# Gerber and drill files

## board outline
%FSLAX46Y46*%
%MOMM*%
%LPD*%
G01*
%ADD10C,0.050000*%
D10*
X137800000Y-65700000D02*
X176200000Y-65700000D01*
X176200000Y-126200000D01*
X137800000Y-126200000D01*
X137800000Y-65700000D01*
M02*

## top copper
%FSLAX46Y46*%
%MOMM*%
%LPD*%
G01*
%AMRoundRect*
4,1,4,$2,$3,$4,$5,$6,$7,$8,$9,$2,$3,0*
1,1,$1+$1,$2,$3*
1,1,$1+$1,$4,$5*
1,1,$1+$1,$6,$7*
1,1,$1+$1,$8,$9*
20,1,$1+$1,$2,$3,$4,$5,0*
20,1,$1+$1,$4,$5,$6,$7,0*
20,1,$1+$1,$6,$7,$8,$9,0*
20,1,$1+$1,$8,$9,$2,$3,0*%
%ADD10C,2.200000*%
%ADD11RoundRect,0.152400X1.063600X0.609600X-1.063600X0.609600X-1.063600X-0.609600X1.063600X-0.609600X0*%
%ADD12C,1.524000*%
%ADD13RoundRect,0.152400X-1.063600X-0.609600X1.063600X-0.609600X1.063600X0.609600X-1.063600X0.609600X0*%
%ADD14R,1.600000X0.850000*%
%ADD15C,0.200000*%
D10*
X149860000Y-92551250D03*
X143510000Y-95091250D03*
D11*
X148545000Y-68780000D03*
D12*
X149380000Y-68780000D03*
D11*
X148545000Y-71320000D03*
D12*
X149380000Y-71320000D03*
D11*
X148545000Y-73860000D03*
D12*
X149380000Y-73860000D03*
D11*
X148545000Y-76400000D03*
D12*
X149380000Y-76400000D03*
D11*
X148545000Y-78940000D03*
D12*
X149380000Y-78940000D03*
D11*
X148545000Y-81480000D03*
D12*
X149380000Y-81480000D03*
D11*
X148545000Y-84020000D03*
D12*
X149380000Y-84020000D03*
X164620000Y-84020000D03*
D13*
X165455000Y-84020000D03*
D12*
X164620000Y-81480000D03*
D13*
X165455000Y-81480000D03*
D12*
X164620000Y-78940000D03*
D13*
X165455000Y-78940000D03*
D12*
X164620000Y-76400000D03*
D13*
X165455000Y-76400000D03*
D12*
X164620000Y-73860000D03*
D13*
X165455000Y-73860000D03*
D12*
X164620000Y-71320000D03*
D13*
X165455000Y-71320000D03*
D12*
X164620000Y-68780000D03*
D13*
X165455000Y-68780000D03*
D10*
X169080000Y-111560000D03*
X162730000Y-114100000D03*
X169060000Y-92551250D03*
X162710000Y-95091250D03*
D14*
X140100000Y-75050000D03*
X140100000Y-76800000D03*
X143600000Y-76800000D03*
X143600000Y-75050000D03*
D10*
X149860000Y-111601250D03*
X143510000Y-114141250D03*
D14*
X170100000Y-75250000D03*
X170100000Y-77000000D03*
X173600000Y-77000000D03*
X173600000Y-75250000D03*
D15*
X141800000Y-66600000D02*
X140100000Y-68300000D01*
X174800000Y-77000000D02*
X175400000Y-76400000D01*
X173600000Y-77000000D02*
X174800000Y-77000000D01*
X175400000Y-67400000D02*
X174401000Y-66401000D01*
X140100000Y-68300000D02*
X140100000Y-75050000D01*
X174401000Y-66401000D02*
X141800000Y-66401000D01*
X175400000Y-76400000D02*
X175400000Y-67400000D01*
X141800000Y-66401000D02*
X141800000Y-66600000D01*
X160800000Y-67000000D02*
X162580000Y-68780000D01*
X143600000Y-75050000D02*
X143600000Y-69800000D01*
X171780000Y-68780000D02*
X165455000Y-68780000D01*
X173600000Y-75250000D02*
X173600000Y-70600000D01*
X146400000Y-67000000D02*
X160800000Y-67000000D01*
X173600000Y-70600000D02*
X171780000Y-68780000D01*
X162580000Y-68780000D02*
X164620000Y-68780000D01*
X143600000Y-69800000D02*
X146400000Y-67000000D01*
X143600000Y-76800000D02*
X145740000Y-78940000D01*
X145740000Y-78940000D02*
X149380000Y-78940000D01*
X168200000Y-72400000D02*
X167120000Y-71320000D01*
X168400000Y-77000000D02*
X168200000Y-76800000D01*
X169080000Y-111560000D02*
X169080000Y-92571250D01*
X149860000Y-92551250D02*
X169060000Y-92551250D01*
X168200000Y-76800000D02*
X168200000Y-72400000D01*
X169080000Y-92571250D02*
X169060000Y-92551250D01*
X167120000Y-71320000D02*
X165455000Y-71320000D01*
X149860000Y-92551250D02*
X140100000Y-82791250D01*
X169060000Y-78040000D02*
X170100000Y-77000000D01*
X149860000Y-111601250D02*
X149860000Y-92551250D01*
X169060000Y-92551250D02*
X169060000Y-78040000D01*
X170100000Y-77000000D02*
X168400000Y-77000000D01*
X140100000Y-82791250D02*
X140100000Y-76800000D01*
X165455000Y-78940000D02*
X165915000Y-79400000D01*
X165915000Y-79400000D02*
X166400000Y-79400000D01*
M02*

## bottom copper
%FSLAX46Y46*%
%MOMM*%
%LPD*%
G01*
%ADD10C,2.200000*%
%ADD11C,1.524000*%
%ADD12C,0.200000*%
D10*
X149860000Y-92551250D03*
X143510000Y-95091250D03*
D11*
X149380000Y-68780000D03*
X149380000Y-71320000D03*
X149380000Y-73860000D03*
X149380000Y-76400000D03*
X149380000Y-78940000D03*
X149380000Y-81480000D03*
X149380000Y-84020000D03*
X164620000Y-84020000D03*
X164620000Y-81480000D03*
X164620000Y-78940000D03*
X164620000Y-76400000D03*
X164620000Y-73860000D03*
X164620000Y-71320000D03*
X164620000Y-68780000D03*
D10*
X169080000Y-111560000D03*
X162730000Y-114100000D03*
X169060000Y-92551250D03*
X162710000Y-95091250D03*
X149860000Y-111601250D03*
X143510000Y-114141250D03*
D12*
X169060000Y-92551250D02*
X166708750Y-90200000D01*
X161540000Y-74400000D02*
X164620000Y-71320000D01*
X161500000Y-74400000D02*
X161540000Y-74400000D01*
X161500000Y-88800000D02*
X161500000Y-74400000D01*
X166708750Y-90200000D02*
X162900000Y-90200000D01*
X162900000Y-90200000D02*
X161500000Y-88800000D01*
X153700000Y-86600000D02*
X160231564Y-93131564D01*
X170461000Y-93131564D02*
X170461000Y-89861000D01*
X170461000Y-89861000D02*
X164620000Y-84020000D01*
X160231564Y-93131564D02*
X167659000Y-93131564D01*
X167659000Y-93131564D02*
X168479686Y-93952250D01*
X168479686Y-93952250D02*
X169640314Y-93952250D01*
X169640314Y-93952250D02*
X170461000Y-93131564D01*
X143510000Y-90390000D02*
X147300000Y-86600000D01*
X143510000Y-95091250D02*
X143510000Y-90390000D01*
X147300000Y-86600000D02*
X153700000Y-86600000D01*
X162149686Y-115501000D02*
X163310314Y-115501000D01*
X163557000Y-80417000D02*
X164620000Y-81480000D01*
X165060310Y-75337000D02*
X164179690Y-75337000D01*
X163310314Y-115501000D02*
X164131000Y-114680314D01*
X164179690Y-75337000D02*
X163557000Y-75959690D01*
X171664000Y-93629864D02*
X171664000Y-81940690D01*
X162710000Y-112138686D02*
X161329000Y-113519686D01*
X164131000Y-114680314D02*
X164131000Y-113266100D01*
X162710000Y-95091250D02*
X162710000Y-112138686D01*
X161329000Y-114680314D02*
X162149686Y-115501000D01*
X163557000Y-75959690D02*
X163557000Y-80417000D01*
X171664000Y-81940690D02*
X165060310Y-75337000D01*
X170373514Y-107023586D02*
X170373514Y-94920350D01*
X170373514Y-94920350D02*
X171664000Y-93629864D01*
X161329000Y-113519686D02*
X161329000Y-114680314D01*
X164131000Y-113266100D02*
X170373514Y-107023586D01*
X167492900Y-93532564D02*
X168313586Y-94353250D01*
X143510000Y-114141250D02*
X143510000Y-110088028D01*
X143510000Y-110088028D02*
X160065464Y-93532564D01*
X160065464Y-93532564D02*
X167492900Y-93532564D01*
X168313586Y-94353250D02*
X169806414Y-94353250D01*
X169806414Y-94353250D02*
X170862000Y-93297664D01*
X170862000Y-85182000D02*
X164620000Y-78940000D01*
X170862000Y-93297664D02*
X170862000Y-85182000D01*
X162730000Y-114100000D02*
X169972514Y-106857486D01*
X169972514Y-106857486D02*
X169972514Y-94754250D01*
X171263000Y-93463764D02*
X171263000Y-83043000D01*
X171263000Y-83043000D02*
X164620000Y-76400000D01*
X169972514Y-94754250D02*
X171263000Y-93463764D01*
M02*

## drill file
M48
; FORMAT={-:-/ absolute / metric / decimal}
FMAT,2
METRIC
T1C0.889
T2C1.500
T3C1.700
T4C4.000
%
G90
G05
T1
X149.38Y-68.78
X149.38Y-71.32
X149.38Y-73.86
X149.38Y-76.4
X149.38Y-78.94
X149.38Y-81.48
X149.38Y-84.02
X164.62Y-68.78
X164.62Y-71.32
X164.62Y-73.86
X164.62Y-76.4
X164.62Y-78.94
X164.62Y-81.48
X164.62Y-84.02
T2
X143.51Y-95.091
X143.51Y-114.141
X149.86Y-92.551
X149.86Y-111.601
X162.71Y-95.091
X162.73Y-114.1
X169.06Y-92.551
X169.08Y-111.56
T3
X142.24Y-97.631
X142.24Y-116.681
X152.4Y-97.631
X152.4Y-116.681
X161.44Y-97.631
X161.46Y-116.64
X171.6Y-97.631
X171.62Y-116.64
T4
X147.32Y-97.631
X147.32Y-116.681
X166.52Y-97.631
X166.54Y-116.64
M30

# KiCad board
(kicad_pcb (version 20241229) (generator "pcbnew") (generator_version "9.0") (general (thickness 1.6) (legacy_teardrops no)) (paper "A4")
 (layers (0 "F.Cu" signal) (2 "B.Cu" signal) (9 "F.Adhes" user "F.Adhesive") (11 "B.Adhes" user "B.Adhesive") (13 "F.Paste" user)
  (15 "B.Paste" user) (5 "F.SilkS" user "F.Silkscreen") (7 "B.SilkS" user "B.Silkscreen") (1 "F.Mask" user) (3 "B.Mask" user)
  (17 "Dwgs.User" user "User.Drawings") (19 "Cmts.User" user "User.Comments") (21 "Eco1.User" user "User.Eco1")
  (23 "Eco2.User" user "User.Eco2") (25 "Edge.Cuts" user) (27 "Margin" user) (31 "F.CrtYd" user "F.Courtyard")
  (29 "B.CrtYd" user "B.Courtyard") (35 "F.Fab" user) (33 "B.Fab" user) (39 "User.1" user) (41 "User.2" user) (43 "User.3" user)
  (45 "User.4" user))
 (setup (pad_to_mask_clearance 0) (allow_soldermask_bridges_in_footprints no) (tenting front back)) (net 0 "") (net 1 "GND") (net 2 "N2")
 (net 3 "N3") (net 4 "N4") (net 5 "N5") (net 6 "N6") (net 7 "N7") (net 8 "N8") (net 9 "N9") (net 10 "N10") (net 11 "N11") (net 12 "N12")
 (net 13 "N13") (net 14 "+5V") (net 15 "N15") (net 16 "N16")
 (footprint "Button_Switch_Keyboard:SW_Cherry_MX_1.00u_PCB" (layer "F.Cu") (at 149.86 92.55125)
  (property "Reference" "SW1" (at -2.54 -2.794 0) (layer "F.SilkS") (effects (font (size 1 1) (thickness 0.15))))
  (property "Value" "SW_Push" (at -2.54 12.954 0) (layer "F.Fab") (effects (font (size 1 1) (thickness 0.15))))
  (pad "" np_thru_hole circle (at -7.62 5.08) (size 1.7 1.7) (drill 1.7) (layers "*.Cu" "*.Mask"))
  (pad "" np_thru_hole circle (at -2.54 5.08) (size 4 4) (drill 4) (layers "*.Cu" "*.Mask"))
  (pad "" np_thru_hole circle (at 2.54 5.08) (size 1.7 1.7) (drill 1.7) (layers "*.Cu" "*.Mask"))
  (pad "1" thru_hole circle (at 0 0) (size 2.2 2.2) (drill 1.5) (layers "*.Cu" "*.Mask") (remove_unused_layers no) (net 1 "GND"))
  (pad "2" thru_hole circle (at -6.35 2.54) (size 2.2 2.2) (drill 1.5) (layers "*.Cu" "*.Mask") (remove_unused_layers no) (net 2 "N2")))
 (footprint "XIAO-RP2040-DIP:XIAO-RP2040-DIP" (layer "F.Cu") (at 157 76.4)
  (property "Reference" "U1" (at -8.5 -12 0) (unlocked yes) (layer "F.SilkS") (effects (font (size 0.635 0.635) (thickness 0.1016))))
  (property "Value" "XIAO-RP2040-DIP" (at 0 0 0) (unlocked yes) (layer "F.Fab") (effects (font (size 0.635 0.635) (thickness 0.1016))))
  (pad "1" smd roundrect (at -8.455 -7.62 180) (size 2.432 1.524) (layers "F.Cu" "F.Mask") (roundrect_rratio 0.1) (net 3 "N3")
   (thermal_bridge_angle 45))
  (pad "1" thru_hole circle (at -7.62 -7.62 180) (size 1.524 1.524) (drill 0.889) (layers "*.Cu" "*.Mask") (remove_unused_layers no)
   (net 3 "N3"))
  (pad "2" smd roundrect (at -8.455 -5.08 180) (size 2.432 1.524) (layers "F.Cu" "F.Mask") (roundrect_rratio 0.1) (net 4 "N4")
   (thermal_bridge_angle 45))
  (pad "2" thru_hole circle (at -7.62 -5.08 180) (size 1.524 1.524) (drill 0.889) (layers "*.Cu" "*.Mask") (remove_unused_layers no)
   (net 4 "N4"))
  (pad "3" smd roundrect (at -8.455 -2.54 180) (size 2.432 1.524) (layers "F.Cu" "F.Mask") (roundrect_rratio 0.1) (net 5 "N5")
   (thermal_bridge_angle 45))
  (pad "3" thru_hole circle (at -7.62 -2.54 180) (size 1.524 1.524) (drill 0.889) (layers "*.Cu" "*.Mask") (remove_unused_layers no)
   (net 5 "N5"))
  (pad "4" smd roundrect (at -8.455 0 180) (size 2.432 1.524) (layers "F.Cu" "F.Mask") (roundrect_rratio 0.1) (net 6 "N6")
   (thermal_bridge_angle 45))
  (pad "4" thru_hole circle (at -7.62 0 180) (size 1.524 1.524) (drill 0.889) (layers "*.Cu" "*.Mask") (remove_unused_layers no)
   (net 6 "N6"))
  (pad "5" smd roundrect (at -8.455 2.54 180) (size 2.432 1.524) (layers "F.Cu" "F.Mask") (roundrect_rratio 0.1) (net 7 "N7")
   (thermal_bridge_angle 45))
  (pad "5" thru_hole circle (at -7.62 2.54 180) (size 1.524 1.524) (drill 0.889) (layers "*.Cu" "*.Mask") (remove_unused_layers no)
   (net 7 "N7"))
  (pad "6" smd roundrect (at -8.455 5.08 180) (size 2.432 1.524) (layers "F.Cu" "F.Mask") (roundrect_rratio 0.1) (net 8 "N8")
   (thermal_bridge_angle 45))
  (pad "6" thru_hole circle (at -7.62 5.08 180) (size 1.524 1.524) (drill 0.889) (layers "*.Cu" "*.Mask") (remove_unused_layers no)
   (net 8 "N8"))
  (pad "7" smd roundrect (at -8.455 7.62 180) (size 2.432 1.524) (layers "F.Cu" "F.Mask") (roundrect_rratio 0.1) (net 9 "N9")
   (thermal_bridge_angle 45))
  (pad "7" thru_hole circle (at -7.62 7.62 180) (size 1.524 1.524) (drill 0.889) (layers "*.Cu" "*.Mask") (remove_unused_layers no)
   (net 9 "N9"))
  (pad "8" thru_hole circle (at 7.62 7.62) (size 1.524 1.524) (drill 0.889) (layers "*.Cu" "*.Mask") (remove_unused_layers no) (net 2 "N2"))
  (pad "8" smd roundrect (at 8.455 7.62) (size 2.432 1.524) (layers "F.Cu" "F.Mask") (roundrect_rratio 0.1) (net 2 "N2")
   (thermal_bridge_angle 45))
  (pad "9" thru_hole circle (at 7.62 5.08) (size 1.524 1.524) (drill 0.889) (layers "*.Cu" "*.Mask") (remove_unused_layers no)
   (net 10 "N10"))
  (pad "9" smd roundrect (at 8.455 5.08) (size 2.432 1.524) (layers "F.Cu" "F.Mask") (roundrect_rratio 0.1) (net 10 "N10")
   (thermal_bridge_angle 45))
  (pad "10" thru_hole circle (at 7.62 2.54) (size 1.524 1.524) (drill 0.889) (layers "*.Cu" "*.Mask") (remove_unused_layers no)
   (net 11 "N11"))
  (pad "10" smd roundrect (at 8.455 2.54) (size 2.432 1.524) (layers "F.Cu" "F.Mask") (roundrect_rratio 0.1) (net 11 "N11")
   (thermal_bridge_angle 45))
  (pad "11" thru_hole circle (at 7.62 0) (size 1.524 1.524) (drill 0.889) (layers "*.Cu" "*.Mask") (remove_unused_layers no) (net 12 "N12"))
  (pad "11" smd roundrect (at 8.455 0) (size 2.432 1.524) (layers "F.Cu" "F.Mask") (roundrect_rratio 0.1) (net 12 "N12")
   (thermal_bridge_angle 45))
  (pad "12" thru_hole circle (at 7.62 -2.54) (size 1.524 1.524) (drill 0.889) (layers "*.Cu" "*.Mask") (remove_unused_layers no)
   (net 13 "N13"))
  (pad "12" smd roundrect (at 8.455 -2.54) (size 2.432 1.524) (layers "F.Cu" "F.Mask") (roundrect_rratio 0.1) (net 13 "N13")
   (thermal_bridge_angle 45))
  (pad "13" thru_hole circle (at 7.62 -5.08) (size 1.524 1.524) (drill 0.889) (layers "*.Cu" "*.Mask") (remove_unused_layers no)
   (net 1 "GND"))
  (pad "13" smd roundrect (at 8.455 -5.08) (size 2.432 1.524) (layers "F.Cu" "F.Mask") (roundrect_rratio 0.1) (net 1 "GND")
   (thermal_bridge_angle 45))
  (pad "14" thru_hole circle (at 7.62 -7.62) (size 1.524 1.524) (drill 0.889) (layers "*.Cu" "*.Mask") (remove_unused_layers no)
   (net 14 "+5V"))
  (pad "14" smd roundrect (at 8.455 -7.62) (size 2.432 1.524) (layers "F.Cu" "F.Mask") (roundrect_rratio 0.1) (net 14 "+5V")
   (thermal_bridge_angle 45)))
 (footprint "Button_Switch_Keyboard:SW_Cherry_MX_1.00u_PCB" (layer "F.Cu") (at 169.08 111.56)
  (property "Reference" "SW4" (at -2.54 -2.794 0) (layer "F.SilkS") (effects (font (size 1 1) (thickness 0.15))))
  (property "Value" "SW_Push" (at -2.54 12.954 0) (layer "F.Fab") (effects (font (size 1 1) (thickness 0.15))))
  (pad "" np_thru_hole circle (at -7.62 5.08) (size 1.7 1.7) (drill 1.7) (layers "*.Cu" "*.Mask"))
  (pad "" np_thru_hole circle (at -2.54 5.08) (size 4 4) (drill 4) (layers "*.Cu" "*.Mask"))
  (pad "" np_thru_hole circle (at 2.54 5.08) (size 1.7 1.7) (drill 1.7) (layers "*.Cu" "*.Mask"))
  (pad "1" thru_hole circle (at 0 0) (size 2.2 2.2) (drill 1.5) (layers "*.Cu" "*.Mask") (remove_unused_layers no) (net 1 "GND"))
  (pad "2" thru_hole circle (at -6.35 2.54) (size 2.2 2.2) (drill 1.5) (layers "*.Cu" "*.Mask") (remove_unused_layers no) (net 12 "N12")))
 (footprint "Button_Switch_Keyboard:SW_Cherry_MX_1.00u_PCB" (layer "F.Cu") (at 169.06 92.55125)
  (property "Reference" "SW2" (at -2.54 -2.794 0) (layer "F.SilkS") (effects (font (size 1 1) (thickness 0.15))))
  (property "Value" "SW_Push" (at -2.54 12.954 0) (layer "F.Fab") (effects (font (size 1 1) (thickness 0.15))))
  (pad "" np_thru_hole circle (at -7.62 5.08) (size 1.7 1.7) (drill 1.7) (layers "*.Cu" "*.Mask"))
  (pad "" np_thru_hole circle (at -2.54 5.08) (size 4 4) (drill 4) (layers "*.Cu" "*.Mask"))
  (pad "" np_thru_hole circle (at 2.54 5.08) (size 1.7 1.7) (drill 1.7) (layers "*.Cu" "*.Mask"))
  (pad "1" thru_hole circle (at 0 0) (size 2.2 2.2) (drill 1.5) (layers "*.Cu" "*.Mask") (remove_unused_layers no) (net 1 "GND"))
  (pad "2" thru_hole circle (at -6.35 2.54) (size 2.2 2.2) (drill 1.5) (layers "*.Cu" "*.Mask") (remove_unused_layers no) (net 10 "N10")))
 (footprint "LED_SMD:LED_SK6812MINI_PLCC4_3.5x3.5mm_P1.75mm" (layer "F.Cu") (at 141.85 75.925)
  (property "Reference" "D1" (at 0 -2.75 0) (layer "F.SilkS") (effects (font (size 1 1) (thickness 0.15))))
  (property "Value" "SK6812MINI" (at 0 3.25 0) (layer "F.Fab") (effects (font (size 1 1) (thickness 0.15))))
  (pad "1" smd rect (at -1.75 -0.875) (size 1.6 0.85) (layers "F.Cu" "F.Mask" "F.Paste") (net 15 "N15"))
  (pad "2" smd rect (at -1.75 0.875) (size 1.6 0.85) (layers "F.Cu" "F.Mask" "F.Paste") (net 1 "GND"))
  (pad "3" smd rect (at 1.75 0.875) (size 1.6 0.85) (layers "F.Cu" "F.Mask" "F.Paste") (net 7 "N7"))
  (pad "4" smd rect (at 1.75 -0.875) (size 1.6 0.85) (layers "F.Cu" "F.Mask" "F.Paste") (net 14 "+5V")))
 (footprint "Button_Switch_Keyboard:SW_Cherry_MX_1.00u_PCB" (layer "F.Cu") (at 149.86 111.60125)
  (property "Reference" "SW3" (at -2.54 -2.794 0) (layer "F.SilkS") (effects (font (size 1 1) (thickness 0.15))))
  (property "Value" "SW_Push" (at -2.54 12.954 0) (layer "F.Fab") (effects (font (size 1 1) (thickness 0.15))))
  (pad "" np_thru_hole circle (at -7.62 5.08) (size 1.7 1.7) (drill 1.7) (layers "*.Cu" "*.Mask"))
  (pad "" np_thru_hole circle (at -2.54 5.08) (size 4 4) (drill 4) (layers "*.Cu" "*.Mask"))
  (pad "" np_thru_hole circle (at 2.54 5.08) (size 1.7 1.7) (drill 1.7) (layers "*.Cu" "*.Mask"))
  (pad "1" thru_hole circle (at 0 0) (size 2.2 2.2) (drill 1.5) (layers "*.Cu" "*.Mask") (remove_unused_layers no) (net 1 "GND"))
  (pad "2" thru_hole circle (at -6.35 2.54) (size 2.2 2.2) (drill 1.5) (layers "*.Cu" "*.Mask") (remove_unused_layers no) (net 11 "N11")))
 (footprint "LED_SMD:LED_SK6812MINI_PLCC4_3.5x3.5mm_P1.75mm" (layer "F.Cu") (at 171.85 76.125)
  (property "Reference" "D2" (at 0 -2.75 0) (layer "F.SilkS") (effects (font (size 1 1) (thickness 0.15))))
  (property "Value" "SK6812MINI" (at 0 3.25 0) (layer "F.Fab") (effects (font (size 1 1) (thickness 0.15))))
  (pad "1" smd rect (at -1.75 -0.875) (size 1.6 0.85) (layers "F.Cu" "F.Mask" "F.Paste") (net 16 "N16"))
  (pad "2" smd rect (at -1.75 0.875) (size 1.6 0.85) (layers "F.Cu" "F.Mask" "F.Paste") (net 1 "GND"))
  (pad "3" smd rect (at 1.75 0.875) (size 1.6 0.85) (layers "F.Cu" "F.Mask" "F.Paste") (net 15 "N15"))
  (pad "4" smd rect (at 1.75 -0.875) (size 1.6 0.85) (layers "F.Cu" "F.Mask" "F.Paste") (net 14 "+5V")))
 (gr_rect (start 137.8 65.7) (end 176.2 126.2) (stroke (width 0.05) (type default)) (fill no) (layer "Edge.Cuts"))
 (segment (start 141.8 66.6) (end 140.1 68.3) (width 0.2) (layer "F.Cu") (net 15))
 (segment (start 174.8 77) (end 175.4 76.4) (width 0.2) (layer "F.Cu") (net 15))
 (segment (start 173.6 77) (end 174.8 77) (width 0.2) (layer "F.Cu") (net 15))
 (segment (start 175.4 67.4) (end 174.401 66.401) (width 0.2) (layer "F.Cu") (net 15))
 (segment (start 140.1 68.3) (end 140.1 75.05) (width 0.2) (layer "F.Cu") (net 15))
 (segment (start 174.401 66.401) (end 141.8 66.401) (width 0.2) (layer "F.Cu") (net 15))
 (segment (start 175.4 76.4) (end 175.4 67.4) (width 0.2) (layer "F.Cu") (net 15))
 (segment (start 141.8 66.401) (end 141.8 66.6) (width 0.2) (layer "F.Cu") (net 15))
 (segment (start 160.8 67) (end 162.58 68.78) (width 0.2) (layer "F.Cu") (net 14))
 (segment (start 143.6 75.05) (end 143.6 69.8) (width 0.2) (layer "F.Cu") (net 14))
 (segment (start 171.78 68.78) (end 165.455 68.78) (width 0.2) (layer "F.Cu") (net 14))
 (segment (start 173.6 75.25) (end 173.6 70.6) (width 0.2) (layer "F.Cu") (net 14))
 (segment (start 146.4 67) (end 160.8 67) (width 0.2) (layer "F.Cu") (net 14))
 (segment (start 173.6 70.6) (end 171.78 68.78) (width 0.2) (layer "F.Cu") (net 14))
 (segment (start 162.58 68.78) (end 164.62 68.78) (width 0.2) (layer "F.Cu") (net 14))
 (segment (start 143.6 69.8) (end 146.4 67) (width 0.2) (layer "F.Cu") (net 14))
 (segment (start 143.6 76.8) (end 145.74 78.94) (width 0.2) (layer "F.Cu") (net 7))
 (segment (start 145.74 78.94) (end 149.38 78.94) (width 0.2) (layer "F.Cu") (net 7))
 (segment (start 168.2 72.4) (end 167.12 71.32) (width 0.2) (layer "F.Cu") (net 1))
 (segment (start 168.4 77) (end 168.2 76.8) (width 0.2) (layer "F.Cu") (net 1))
 (segment (start 169.08 111.56) (end 169.08 92.57125) (width 0.2) (layer "F.Cu") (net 1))
 (segment (start 149.86 92.55125) (end 169.06 92.55125) (width 0.2) (layer "F.Cu") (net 1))
 (segment (start 168.2 76.8) (end 168.2 72.4) (width 0.2) (layer "F.Cu") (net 1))
 (segment (start 169.08 92.57125) (end 169.06 92.55125) (width 0.2) (layer "F.Cu") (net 1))
 (segment (start 167.12 71.32) (end 165.455 71.32) (width 0.2) (layer "F.Cu") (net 1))
 (segment (start 149.86 92.55125) (end 140.1 82.79125) (width 0.2) (layer "F.Cu") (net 1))
 (segment (start 169.06 78.04) (end 170.1 77) (width 0.2) (layer "F.Cu") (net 1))
 (segment (start 149.86 111.60125) (end 149.86 92.55125) (width 0.2) (layer "F.Cu") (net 1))
 (segment (start 169.06 92.55125) (end 169.06 78.04) (width 0.2) (layer "F.Cu") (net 1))
 (segment (start 170.1 77) (end 168.4 77) (width 0.2) (layer "F.Cu") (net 1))
 (segment (start 140.1 82.79125) (end 140.1 76.8) (width 0.2) (layer "F.Cu") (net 1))
 (segment (start 169.06 92.55125) (end 166.70875 90.2) (width 0.2) (layer "B.Cu") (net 1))
 (segment (start 161.54 74.4) (end 164.62 71.32) (width 0.2) (layer "B.Cu") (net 1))
 (segment (start 161.5 74.4) (end 161.54 74.4) (width 0.2) (layer "B.Cu") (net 1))
 (segment (start 161.5 88.8) (end 161.5 74.4) (width 0.2) (layer "B.Cu") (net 1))
 (segment (start 166.70875 90.2) (end 162.9 90.2) (width 0.2) (layer "B.Cu") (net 1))
 (segment (start 162.9 90.2) (end 161.5 88.8) (width 0.2) (layer "B.Cu") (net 1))
 (segment (start 153.7 86.6) (end 160.231564 93.131564) (width 0.2) (layer "B.Cu") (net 2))
 (segment (start 170.461 93.131564) (end 170.461 89.861) (width 0.2) (layer "B.Cu") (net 2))
 (segment (start 170.461 89.861) (end 164.62 84.02) (width 0.2) (layer "B.Cu") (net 2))
 (segment (start 160.231564 93.131564) (end 167.659 93.131564) (width 0.2) (layer "B.Cu") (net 2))
 (segment (start 167.659 93.131564) (end 168.479686 93.95225) (width 0.2) (layer "B.Cu") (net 2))
 (segment (start 168.479686 93.95225) (end 169.640314 93.95225) (width 0.2) (layer "B.Cu") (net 2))
 (segment (start 169.640314 93.95225) (end 170.461 93.131564) (width 0.2) (layer "B.Cu") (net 2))
 (segment (start 143.51 90.39) (end 147.3 86.6) (width 0.2) (layer "B.Cu") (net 2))
 (segment (start 143.51 95.09125) (end 143.51 90.39) (width 0.2) (layer "B.Cu") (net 2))
 (segment (start 147.3 86.6) (end 153.7 86.6) (width 0.2) (layer "B.Cu") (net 2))
 (segment (start 162.149686 115.501) (end 163.310314 115.501) (width 0.2) (layer "B.Cu") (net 10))
 (segment (start 163.557 80.417) (end 164.62 81.48) (width 0.2) (layer "B.Cu") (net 10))
 (segment (start 165.06031 75.337) (end 164.17969 75.337) (width 0.2) (layer "B.Cu") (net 10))
 (segment (start 163.310314 115.501) (end 164.131 114.680314) (width 0.2) (layer "B.Cu") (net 10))
 (segment (start 164.17969 75.337) (end 163.557 75.95969) (width 0.2) (layer "B.Cu") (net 10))
 (segment (start 171.664 93.629864) (end 171.664 81.94069) (width 0.2) (layer "B.Cu") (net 10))
 (segment (start 162.71 112.138686) (end 161.329 113.519686) (width 0.2) (layer "B.Cu") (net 10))
 (segment (start 164.131 114.680314) (end 164.131 113.2661) (width 0.2) (layer "B.Cu") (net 10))
 (segment (start 162.71 95.09125) (end 162.71 112.138686) (width 0.2) (layer "B.Cu") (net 10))
 (segment (start 161.329 114.680314) (end 162.149686 115.501) (width 0.2) (layer "B.Cu") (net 10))
 (segment (start 163.557 75.95969) (end 163.557 80.417) (width 0.2) (layer "B.Cu") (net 10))
 (segment (start 171.664 81.94069) (end 165.06031 75.337) (width 0.2) (layer "B.Cu") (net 10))
 (segment (start 170.373514 107.023586) (end 170.373514 94.92035) (width 0.2) (layer "B.Cu") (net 10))
 (segment (start 170.373514 94.92035) (end 171.664 93.629864) (width 0.2) (layer "B.Cu") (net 10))
 (segment (start 161.329 113.519686) (end 161.329 114.680314) (width 0.2) (layer "B.Cu") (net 10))
 (segment (start 164.131 113.2661) (end 170.373514 107.023586) (width 0.2) (layer "B.Cu") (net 10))
 (segment (start 165.455 78.94) (end 165.915 79.4) (width 0.2) (layer "F.Cu") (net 11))
 (segment (start 165.915 79.4) (end 166.4 79.4) (width 0.2) (layer "F.Cu") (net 11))
 (segment (start 167.4929 93.532564) (end 168.313586 94.35325) (width 0.2) (layer "B.Cu") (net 11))
 (segment (start 143.51 114.14125) (end 143.51 110.088028) (width 0.2) (layer "B.Cu") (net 11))
 (segment (start 143.51 110.088028) (end 160.065464 93.532564) (width 0.2) (layer "B.Cu") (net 11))
 (segment (start 160.065464 93.532564) (end 167.4929 93.532564) (width 0.2) (layer "B.Cu") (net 11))
 (segment (start 168.313586 94.35325) (end 169.806414 94.35325) (width 0.2) (layer "B.Cu") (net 11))
 (segment (start 169.806414 94.35325) (end 170.862 93.297664) (width 0.2) (layer "B.Cu") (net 11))
 (segment (start 170.862 85.182) (end 164.62 78.94) (width 0.2) (layer "B.Cu") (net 11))
 (segment (start 170.862 93.297664) (end 170.862 85.182) (width 0.2) (layer "B.Cu") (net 11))
 (segment (start 162.73 114.1) (end 169.972514 106.857486) (width 0.2) (layer "B.Cu") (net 12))
 (segment (start 169.972514 106.857486) (end 169.972514 94.75425) (width 0.2) (layer "B.Cu") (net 12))
 (segment (start 171.263 93.463764) (end 171.263 83.043) (width 0.2) (layer "B.Cu") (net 12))
 (segment (start 171.263 83.043) (end 164.62 76.4) (width 0.2) (layer "B.Cu") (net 12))
 (segment (start 169.972514 94.75425) (end 171.263 93.463764) (width 0.2) (layer "B.Cu") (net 12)))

